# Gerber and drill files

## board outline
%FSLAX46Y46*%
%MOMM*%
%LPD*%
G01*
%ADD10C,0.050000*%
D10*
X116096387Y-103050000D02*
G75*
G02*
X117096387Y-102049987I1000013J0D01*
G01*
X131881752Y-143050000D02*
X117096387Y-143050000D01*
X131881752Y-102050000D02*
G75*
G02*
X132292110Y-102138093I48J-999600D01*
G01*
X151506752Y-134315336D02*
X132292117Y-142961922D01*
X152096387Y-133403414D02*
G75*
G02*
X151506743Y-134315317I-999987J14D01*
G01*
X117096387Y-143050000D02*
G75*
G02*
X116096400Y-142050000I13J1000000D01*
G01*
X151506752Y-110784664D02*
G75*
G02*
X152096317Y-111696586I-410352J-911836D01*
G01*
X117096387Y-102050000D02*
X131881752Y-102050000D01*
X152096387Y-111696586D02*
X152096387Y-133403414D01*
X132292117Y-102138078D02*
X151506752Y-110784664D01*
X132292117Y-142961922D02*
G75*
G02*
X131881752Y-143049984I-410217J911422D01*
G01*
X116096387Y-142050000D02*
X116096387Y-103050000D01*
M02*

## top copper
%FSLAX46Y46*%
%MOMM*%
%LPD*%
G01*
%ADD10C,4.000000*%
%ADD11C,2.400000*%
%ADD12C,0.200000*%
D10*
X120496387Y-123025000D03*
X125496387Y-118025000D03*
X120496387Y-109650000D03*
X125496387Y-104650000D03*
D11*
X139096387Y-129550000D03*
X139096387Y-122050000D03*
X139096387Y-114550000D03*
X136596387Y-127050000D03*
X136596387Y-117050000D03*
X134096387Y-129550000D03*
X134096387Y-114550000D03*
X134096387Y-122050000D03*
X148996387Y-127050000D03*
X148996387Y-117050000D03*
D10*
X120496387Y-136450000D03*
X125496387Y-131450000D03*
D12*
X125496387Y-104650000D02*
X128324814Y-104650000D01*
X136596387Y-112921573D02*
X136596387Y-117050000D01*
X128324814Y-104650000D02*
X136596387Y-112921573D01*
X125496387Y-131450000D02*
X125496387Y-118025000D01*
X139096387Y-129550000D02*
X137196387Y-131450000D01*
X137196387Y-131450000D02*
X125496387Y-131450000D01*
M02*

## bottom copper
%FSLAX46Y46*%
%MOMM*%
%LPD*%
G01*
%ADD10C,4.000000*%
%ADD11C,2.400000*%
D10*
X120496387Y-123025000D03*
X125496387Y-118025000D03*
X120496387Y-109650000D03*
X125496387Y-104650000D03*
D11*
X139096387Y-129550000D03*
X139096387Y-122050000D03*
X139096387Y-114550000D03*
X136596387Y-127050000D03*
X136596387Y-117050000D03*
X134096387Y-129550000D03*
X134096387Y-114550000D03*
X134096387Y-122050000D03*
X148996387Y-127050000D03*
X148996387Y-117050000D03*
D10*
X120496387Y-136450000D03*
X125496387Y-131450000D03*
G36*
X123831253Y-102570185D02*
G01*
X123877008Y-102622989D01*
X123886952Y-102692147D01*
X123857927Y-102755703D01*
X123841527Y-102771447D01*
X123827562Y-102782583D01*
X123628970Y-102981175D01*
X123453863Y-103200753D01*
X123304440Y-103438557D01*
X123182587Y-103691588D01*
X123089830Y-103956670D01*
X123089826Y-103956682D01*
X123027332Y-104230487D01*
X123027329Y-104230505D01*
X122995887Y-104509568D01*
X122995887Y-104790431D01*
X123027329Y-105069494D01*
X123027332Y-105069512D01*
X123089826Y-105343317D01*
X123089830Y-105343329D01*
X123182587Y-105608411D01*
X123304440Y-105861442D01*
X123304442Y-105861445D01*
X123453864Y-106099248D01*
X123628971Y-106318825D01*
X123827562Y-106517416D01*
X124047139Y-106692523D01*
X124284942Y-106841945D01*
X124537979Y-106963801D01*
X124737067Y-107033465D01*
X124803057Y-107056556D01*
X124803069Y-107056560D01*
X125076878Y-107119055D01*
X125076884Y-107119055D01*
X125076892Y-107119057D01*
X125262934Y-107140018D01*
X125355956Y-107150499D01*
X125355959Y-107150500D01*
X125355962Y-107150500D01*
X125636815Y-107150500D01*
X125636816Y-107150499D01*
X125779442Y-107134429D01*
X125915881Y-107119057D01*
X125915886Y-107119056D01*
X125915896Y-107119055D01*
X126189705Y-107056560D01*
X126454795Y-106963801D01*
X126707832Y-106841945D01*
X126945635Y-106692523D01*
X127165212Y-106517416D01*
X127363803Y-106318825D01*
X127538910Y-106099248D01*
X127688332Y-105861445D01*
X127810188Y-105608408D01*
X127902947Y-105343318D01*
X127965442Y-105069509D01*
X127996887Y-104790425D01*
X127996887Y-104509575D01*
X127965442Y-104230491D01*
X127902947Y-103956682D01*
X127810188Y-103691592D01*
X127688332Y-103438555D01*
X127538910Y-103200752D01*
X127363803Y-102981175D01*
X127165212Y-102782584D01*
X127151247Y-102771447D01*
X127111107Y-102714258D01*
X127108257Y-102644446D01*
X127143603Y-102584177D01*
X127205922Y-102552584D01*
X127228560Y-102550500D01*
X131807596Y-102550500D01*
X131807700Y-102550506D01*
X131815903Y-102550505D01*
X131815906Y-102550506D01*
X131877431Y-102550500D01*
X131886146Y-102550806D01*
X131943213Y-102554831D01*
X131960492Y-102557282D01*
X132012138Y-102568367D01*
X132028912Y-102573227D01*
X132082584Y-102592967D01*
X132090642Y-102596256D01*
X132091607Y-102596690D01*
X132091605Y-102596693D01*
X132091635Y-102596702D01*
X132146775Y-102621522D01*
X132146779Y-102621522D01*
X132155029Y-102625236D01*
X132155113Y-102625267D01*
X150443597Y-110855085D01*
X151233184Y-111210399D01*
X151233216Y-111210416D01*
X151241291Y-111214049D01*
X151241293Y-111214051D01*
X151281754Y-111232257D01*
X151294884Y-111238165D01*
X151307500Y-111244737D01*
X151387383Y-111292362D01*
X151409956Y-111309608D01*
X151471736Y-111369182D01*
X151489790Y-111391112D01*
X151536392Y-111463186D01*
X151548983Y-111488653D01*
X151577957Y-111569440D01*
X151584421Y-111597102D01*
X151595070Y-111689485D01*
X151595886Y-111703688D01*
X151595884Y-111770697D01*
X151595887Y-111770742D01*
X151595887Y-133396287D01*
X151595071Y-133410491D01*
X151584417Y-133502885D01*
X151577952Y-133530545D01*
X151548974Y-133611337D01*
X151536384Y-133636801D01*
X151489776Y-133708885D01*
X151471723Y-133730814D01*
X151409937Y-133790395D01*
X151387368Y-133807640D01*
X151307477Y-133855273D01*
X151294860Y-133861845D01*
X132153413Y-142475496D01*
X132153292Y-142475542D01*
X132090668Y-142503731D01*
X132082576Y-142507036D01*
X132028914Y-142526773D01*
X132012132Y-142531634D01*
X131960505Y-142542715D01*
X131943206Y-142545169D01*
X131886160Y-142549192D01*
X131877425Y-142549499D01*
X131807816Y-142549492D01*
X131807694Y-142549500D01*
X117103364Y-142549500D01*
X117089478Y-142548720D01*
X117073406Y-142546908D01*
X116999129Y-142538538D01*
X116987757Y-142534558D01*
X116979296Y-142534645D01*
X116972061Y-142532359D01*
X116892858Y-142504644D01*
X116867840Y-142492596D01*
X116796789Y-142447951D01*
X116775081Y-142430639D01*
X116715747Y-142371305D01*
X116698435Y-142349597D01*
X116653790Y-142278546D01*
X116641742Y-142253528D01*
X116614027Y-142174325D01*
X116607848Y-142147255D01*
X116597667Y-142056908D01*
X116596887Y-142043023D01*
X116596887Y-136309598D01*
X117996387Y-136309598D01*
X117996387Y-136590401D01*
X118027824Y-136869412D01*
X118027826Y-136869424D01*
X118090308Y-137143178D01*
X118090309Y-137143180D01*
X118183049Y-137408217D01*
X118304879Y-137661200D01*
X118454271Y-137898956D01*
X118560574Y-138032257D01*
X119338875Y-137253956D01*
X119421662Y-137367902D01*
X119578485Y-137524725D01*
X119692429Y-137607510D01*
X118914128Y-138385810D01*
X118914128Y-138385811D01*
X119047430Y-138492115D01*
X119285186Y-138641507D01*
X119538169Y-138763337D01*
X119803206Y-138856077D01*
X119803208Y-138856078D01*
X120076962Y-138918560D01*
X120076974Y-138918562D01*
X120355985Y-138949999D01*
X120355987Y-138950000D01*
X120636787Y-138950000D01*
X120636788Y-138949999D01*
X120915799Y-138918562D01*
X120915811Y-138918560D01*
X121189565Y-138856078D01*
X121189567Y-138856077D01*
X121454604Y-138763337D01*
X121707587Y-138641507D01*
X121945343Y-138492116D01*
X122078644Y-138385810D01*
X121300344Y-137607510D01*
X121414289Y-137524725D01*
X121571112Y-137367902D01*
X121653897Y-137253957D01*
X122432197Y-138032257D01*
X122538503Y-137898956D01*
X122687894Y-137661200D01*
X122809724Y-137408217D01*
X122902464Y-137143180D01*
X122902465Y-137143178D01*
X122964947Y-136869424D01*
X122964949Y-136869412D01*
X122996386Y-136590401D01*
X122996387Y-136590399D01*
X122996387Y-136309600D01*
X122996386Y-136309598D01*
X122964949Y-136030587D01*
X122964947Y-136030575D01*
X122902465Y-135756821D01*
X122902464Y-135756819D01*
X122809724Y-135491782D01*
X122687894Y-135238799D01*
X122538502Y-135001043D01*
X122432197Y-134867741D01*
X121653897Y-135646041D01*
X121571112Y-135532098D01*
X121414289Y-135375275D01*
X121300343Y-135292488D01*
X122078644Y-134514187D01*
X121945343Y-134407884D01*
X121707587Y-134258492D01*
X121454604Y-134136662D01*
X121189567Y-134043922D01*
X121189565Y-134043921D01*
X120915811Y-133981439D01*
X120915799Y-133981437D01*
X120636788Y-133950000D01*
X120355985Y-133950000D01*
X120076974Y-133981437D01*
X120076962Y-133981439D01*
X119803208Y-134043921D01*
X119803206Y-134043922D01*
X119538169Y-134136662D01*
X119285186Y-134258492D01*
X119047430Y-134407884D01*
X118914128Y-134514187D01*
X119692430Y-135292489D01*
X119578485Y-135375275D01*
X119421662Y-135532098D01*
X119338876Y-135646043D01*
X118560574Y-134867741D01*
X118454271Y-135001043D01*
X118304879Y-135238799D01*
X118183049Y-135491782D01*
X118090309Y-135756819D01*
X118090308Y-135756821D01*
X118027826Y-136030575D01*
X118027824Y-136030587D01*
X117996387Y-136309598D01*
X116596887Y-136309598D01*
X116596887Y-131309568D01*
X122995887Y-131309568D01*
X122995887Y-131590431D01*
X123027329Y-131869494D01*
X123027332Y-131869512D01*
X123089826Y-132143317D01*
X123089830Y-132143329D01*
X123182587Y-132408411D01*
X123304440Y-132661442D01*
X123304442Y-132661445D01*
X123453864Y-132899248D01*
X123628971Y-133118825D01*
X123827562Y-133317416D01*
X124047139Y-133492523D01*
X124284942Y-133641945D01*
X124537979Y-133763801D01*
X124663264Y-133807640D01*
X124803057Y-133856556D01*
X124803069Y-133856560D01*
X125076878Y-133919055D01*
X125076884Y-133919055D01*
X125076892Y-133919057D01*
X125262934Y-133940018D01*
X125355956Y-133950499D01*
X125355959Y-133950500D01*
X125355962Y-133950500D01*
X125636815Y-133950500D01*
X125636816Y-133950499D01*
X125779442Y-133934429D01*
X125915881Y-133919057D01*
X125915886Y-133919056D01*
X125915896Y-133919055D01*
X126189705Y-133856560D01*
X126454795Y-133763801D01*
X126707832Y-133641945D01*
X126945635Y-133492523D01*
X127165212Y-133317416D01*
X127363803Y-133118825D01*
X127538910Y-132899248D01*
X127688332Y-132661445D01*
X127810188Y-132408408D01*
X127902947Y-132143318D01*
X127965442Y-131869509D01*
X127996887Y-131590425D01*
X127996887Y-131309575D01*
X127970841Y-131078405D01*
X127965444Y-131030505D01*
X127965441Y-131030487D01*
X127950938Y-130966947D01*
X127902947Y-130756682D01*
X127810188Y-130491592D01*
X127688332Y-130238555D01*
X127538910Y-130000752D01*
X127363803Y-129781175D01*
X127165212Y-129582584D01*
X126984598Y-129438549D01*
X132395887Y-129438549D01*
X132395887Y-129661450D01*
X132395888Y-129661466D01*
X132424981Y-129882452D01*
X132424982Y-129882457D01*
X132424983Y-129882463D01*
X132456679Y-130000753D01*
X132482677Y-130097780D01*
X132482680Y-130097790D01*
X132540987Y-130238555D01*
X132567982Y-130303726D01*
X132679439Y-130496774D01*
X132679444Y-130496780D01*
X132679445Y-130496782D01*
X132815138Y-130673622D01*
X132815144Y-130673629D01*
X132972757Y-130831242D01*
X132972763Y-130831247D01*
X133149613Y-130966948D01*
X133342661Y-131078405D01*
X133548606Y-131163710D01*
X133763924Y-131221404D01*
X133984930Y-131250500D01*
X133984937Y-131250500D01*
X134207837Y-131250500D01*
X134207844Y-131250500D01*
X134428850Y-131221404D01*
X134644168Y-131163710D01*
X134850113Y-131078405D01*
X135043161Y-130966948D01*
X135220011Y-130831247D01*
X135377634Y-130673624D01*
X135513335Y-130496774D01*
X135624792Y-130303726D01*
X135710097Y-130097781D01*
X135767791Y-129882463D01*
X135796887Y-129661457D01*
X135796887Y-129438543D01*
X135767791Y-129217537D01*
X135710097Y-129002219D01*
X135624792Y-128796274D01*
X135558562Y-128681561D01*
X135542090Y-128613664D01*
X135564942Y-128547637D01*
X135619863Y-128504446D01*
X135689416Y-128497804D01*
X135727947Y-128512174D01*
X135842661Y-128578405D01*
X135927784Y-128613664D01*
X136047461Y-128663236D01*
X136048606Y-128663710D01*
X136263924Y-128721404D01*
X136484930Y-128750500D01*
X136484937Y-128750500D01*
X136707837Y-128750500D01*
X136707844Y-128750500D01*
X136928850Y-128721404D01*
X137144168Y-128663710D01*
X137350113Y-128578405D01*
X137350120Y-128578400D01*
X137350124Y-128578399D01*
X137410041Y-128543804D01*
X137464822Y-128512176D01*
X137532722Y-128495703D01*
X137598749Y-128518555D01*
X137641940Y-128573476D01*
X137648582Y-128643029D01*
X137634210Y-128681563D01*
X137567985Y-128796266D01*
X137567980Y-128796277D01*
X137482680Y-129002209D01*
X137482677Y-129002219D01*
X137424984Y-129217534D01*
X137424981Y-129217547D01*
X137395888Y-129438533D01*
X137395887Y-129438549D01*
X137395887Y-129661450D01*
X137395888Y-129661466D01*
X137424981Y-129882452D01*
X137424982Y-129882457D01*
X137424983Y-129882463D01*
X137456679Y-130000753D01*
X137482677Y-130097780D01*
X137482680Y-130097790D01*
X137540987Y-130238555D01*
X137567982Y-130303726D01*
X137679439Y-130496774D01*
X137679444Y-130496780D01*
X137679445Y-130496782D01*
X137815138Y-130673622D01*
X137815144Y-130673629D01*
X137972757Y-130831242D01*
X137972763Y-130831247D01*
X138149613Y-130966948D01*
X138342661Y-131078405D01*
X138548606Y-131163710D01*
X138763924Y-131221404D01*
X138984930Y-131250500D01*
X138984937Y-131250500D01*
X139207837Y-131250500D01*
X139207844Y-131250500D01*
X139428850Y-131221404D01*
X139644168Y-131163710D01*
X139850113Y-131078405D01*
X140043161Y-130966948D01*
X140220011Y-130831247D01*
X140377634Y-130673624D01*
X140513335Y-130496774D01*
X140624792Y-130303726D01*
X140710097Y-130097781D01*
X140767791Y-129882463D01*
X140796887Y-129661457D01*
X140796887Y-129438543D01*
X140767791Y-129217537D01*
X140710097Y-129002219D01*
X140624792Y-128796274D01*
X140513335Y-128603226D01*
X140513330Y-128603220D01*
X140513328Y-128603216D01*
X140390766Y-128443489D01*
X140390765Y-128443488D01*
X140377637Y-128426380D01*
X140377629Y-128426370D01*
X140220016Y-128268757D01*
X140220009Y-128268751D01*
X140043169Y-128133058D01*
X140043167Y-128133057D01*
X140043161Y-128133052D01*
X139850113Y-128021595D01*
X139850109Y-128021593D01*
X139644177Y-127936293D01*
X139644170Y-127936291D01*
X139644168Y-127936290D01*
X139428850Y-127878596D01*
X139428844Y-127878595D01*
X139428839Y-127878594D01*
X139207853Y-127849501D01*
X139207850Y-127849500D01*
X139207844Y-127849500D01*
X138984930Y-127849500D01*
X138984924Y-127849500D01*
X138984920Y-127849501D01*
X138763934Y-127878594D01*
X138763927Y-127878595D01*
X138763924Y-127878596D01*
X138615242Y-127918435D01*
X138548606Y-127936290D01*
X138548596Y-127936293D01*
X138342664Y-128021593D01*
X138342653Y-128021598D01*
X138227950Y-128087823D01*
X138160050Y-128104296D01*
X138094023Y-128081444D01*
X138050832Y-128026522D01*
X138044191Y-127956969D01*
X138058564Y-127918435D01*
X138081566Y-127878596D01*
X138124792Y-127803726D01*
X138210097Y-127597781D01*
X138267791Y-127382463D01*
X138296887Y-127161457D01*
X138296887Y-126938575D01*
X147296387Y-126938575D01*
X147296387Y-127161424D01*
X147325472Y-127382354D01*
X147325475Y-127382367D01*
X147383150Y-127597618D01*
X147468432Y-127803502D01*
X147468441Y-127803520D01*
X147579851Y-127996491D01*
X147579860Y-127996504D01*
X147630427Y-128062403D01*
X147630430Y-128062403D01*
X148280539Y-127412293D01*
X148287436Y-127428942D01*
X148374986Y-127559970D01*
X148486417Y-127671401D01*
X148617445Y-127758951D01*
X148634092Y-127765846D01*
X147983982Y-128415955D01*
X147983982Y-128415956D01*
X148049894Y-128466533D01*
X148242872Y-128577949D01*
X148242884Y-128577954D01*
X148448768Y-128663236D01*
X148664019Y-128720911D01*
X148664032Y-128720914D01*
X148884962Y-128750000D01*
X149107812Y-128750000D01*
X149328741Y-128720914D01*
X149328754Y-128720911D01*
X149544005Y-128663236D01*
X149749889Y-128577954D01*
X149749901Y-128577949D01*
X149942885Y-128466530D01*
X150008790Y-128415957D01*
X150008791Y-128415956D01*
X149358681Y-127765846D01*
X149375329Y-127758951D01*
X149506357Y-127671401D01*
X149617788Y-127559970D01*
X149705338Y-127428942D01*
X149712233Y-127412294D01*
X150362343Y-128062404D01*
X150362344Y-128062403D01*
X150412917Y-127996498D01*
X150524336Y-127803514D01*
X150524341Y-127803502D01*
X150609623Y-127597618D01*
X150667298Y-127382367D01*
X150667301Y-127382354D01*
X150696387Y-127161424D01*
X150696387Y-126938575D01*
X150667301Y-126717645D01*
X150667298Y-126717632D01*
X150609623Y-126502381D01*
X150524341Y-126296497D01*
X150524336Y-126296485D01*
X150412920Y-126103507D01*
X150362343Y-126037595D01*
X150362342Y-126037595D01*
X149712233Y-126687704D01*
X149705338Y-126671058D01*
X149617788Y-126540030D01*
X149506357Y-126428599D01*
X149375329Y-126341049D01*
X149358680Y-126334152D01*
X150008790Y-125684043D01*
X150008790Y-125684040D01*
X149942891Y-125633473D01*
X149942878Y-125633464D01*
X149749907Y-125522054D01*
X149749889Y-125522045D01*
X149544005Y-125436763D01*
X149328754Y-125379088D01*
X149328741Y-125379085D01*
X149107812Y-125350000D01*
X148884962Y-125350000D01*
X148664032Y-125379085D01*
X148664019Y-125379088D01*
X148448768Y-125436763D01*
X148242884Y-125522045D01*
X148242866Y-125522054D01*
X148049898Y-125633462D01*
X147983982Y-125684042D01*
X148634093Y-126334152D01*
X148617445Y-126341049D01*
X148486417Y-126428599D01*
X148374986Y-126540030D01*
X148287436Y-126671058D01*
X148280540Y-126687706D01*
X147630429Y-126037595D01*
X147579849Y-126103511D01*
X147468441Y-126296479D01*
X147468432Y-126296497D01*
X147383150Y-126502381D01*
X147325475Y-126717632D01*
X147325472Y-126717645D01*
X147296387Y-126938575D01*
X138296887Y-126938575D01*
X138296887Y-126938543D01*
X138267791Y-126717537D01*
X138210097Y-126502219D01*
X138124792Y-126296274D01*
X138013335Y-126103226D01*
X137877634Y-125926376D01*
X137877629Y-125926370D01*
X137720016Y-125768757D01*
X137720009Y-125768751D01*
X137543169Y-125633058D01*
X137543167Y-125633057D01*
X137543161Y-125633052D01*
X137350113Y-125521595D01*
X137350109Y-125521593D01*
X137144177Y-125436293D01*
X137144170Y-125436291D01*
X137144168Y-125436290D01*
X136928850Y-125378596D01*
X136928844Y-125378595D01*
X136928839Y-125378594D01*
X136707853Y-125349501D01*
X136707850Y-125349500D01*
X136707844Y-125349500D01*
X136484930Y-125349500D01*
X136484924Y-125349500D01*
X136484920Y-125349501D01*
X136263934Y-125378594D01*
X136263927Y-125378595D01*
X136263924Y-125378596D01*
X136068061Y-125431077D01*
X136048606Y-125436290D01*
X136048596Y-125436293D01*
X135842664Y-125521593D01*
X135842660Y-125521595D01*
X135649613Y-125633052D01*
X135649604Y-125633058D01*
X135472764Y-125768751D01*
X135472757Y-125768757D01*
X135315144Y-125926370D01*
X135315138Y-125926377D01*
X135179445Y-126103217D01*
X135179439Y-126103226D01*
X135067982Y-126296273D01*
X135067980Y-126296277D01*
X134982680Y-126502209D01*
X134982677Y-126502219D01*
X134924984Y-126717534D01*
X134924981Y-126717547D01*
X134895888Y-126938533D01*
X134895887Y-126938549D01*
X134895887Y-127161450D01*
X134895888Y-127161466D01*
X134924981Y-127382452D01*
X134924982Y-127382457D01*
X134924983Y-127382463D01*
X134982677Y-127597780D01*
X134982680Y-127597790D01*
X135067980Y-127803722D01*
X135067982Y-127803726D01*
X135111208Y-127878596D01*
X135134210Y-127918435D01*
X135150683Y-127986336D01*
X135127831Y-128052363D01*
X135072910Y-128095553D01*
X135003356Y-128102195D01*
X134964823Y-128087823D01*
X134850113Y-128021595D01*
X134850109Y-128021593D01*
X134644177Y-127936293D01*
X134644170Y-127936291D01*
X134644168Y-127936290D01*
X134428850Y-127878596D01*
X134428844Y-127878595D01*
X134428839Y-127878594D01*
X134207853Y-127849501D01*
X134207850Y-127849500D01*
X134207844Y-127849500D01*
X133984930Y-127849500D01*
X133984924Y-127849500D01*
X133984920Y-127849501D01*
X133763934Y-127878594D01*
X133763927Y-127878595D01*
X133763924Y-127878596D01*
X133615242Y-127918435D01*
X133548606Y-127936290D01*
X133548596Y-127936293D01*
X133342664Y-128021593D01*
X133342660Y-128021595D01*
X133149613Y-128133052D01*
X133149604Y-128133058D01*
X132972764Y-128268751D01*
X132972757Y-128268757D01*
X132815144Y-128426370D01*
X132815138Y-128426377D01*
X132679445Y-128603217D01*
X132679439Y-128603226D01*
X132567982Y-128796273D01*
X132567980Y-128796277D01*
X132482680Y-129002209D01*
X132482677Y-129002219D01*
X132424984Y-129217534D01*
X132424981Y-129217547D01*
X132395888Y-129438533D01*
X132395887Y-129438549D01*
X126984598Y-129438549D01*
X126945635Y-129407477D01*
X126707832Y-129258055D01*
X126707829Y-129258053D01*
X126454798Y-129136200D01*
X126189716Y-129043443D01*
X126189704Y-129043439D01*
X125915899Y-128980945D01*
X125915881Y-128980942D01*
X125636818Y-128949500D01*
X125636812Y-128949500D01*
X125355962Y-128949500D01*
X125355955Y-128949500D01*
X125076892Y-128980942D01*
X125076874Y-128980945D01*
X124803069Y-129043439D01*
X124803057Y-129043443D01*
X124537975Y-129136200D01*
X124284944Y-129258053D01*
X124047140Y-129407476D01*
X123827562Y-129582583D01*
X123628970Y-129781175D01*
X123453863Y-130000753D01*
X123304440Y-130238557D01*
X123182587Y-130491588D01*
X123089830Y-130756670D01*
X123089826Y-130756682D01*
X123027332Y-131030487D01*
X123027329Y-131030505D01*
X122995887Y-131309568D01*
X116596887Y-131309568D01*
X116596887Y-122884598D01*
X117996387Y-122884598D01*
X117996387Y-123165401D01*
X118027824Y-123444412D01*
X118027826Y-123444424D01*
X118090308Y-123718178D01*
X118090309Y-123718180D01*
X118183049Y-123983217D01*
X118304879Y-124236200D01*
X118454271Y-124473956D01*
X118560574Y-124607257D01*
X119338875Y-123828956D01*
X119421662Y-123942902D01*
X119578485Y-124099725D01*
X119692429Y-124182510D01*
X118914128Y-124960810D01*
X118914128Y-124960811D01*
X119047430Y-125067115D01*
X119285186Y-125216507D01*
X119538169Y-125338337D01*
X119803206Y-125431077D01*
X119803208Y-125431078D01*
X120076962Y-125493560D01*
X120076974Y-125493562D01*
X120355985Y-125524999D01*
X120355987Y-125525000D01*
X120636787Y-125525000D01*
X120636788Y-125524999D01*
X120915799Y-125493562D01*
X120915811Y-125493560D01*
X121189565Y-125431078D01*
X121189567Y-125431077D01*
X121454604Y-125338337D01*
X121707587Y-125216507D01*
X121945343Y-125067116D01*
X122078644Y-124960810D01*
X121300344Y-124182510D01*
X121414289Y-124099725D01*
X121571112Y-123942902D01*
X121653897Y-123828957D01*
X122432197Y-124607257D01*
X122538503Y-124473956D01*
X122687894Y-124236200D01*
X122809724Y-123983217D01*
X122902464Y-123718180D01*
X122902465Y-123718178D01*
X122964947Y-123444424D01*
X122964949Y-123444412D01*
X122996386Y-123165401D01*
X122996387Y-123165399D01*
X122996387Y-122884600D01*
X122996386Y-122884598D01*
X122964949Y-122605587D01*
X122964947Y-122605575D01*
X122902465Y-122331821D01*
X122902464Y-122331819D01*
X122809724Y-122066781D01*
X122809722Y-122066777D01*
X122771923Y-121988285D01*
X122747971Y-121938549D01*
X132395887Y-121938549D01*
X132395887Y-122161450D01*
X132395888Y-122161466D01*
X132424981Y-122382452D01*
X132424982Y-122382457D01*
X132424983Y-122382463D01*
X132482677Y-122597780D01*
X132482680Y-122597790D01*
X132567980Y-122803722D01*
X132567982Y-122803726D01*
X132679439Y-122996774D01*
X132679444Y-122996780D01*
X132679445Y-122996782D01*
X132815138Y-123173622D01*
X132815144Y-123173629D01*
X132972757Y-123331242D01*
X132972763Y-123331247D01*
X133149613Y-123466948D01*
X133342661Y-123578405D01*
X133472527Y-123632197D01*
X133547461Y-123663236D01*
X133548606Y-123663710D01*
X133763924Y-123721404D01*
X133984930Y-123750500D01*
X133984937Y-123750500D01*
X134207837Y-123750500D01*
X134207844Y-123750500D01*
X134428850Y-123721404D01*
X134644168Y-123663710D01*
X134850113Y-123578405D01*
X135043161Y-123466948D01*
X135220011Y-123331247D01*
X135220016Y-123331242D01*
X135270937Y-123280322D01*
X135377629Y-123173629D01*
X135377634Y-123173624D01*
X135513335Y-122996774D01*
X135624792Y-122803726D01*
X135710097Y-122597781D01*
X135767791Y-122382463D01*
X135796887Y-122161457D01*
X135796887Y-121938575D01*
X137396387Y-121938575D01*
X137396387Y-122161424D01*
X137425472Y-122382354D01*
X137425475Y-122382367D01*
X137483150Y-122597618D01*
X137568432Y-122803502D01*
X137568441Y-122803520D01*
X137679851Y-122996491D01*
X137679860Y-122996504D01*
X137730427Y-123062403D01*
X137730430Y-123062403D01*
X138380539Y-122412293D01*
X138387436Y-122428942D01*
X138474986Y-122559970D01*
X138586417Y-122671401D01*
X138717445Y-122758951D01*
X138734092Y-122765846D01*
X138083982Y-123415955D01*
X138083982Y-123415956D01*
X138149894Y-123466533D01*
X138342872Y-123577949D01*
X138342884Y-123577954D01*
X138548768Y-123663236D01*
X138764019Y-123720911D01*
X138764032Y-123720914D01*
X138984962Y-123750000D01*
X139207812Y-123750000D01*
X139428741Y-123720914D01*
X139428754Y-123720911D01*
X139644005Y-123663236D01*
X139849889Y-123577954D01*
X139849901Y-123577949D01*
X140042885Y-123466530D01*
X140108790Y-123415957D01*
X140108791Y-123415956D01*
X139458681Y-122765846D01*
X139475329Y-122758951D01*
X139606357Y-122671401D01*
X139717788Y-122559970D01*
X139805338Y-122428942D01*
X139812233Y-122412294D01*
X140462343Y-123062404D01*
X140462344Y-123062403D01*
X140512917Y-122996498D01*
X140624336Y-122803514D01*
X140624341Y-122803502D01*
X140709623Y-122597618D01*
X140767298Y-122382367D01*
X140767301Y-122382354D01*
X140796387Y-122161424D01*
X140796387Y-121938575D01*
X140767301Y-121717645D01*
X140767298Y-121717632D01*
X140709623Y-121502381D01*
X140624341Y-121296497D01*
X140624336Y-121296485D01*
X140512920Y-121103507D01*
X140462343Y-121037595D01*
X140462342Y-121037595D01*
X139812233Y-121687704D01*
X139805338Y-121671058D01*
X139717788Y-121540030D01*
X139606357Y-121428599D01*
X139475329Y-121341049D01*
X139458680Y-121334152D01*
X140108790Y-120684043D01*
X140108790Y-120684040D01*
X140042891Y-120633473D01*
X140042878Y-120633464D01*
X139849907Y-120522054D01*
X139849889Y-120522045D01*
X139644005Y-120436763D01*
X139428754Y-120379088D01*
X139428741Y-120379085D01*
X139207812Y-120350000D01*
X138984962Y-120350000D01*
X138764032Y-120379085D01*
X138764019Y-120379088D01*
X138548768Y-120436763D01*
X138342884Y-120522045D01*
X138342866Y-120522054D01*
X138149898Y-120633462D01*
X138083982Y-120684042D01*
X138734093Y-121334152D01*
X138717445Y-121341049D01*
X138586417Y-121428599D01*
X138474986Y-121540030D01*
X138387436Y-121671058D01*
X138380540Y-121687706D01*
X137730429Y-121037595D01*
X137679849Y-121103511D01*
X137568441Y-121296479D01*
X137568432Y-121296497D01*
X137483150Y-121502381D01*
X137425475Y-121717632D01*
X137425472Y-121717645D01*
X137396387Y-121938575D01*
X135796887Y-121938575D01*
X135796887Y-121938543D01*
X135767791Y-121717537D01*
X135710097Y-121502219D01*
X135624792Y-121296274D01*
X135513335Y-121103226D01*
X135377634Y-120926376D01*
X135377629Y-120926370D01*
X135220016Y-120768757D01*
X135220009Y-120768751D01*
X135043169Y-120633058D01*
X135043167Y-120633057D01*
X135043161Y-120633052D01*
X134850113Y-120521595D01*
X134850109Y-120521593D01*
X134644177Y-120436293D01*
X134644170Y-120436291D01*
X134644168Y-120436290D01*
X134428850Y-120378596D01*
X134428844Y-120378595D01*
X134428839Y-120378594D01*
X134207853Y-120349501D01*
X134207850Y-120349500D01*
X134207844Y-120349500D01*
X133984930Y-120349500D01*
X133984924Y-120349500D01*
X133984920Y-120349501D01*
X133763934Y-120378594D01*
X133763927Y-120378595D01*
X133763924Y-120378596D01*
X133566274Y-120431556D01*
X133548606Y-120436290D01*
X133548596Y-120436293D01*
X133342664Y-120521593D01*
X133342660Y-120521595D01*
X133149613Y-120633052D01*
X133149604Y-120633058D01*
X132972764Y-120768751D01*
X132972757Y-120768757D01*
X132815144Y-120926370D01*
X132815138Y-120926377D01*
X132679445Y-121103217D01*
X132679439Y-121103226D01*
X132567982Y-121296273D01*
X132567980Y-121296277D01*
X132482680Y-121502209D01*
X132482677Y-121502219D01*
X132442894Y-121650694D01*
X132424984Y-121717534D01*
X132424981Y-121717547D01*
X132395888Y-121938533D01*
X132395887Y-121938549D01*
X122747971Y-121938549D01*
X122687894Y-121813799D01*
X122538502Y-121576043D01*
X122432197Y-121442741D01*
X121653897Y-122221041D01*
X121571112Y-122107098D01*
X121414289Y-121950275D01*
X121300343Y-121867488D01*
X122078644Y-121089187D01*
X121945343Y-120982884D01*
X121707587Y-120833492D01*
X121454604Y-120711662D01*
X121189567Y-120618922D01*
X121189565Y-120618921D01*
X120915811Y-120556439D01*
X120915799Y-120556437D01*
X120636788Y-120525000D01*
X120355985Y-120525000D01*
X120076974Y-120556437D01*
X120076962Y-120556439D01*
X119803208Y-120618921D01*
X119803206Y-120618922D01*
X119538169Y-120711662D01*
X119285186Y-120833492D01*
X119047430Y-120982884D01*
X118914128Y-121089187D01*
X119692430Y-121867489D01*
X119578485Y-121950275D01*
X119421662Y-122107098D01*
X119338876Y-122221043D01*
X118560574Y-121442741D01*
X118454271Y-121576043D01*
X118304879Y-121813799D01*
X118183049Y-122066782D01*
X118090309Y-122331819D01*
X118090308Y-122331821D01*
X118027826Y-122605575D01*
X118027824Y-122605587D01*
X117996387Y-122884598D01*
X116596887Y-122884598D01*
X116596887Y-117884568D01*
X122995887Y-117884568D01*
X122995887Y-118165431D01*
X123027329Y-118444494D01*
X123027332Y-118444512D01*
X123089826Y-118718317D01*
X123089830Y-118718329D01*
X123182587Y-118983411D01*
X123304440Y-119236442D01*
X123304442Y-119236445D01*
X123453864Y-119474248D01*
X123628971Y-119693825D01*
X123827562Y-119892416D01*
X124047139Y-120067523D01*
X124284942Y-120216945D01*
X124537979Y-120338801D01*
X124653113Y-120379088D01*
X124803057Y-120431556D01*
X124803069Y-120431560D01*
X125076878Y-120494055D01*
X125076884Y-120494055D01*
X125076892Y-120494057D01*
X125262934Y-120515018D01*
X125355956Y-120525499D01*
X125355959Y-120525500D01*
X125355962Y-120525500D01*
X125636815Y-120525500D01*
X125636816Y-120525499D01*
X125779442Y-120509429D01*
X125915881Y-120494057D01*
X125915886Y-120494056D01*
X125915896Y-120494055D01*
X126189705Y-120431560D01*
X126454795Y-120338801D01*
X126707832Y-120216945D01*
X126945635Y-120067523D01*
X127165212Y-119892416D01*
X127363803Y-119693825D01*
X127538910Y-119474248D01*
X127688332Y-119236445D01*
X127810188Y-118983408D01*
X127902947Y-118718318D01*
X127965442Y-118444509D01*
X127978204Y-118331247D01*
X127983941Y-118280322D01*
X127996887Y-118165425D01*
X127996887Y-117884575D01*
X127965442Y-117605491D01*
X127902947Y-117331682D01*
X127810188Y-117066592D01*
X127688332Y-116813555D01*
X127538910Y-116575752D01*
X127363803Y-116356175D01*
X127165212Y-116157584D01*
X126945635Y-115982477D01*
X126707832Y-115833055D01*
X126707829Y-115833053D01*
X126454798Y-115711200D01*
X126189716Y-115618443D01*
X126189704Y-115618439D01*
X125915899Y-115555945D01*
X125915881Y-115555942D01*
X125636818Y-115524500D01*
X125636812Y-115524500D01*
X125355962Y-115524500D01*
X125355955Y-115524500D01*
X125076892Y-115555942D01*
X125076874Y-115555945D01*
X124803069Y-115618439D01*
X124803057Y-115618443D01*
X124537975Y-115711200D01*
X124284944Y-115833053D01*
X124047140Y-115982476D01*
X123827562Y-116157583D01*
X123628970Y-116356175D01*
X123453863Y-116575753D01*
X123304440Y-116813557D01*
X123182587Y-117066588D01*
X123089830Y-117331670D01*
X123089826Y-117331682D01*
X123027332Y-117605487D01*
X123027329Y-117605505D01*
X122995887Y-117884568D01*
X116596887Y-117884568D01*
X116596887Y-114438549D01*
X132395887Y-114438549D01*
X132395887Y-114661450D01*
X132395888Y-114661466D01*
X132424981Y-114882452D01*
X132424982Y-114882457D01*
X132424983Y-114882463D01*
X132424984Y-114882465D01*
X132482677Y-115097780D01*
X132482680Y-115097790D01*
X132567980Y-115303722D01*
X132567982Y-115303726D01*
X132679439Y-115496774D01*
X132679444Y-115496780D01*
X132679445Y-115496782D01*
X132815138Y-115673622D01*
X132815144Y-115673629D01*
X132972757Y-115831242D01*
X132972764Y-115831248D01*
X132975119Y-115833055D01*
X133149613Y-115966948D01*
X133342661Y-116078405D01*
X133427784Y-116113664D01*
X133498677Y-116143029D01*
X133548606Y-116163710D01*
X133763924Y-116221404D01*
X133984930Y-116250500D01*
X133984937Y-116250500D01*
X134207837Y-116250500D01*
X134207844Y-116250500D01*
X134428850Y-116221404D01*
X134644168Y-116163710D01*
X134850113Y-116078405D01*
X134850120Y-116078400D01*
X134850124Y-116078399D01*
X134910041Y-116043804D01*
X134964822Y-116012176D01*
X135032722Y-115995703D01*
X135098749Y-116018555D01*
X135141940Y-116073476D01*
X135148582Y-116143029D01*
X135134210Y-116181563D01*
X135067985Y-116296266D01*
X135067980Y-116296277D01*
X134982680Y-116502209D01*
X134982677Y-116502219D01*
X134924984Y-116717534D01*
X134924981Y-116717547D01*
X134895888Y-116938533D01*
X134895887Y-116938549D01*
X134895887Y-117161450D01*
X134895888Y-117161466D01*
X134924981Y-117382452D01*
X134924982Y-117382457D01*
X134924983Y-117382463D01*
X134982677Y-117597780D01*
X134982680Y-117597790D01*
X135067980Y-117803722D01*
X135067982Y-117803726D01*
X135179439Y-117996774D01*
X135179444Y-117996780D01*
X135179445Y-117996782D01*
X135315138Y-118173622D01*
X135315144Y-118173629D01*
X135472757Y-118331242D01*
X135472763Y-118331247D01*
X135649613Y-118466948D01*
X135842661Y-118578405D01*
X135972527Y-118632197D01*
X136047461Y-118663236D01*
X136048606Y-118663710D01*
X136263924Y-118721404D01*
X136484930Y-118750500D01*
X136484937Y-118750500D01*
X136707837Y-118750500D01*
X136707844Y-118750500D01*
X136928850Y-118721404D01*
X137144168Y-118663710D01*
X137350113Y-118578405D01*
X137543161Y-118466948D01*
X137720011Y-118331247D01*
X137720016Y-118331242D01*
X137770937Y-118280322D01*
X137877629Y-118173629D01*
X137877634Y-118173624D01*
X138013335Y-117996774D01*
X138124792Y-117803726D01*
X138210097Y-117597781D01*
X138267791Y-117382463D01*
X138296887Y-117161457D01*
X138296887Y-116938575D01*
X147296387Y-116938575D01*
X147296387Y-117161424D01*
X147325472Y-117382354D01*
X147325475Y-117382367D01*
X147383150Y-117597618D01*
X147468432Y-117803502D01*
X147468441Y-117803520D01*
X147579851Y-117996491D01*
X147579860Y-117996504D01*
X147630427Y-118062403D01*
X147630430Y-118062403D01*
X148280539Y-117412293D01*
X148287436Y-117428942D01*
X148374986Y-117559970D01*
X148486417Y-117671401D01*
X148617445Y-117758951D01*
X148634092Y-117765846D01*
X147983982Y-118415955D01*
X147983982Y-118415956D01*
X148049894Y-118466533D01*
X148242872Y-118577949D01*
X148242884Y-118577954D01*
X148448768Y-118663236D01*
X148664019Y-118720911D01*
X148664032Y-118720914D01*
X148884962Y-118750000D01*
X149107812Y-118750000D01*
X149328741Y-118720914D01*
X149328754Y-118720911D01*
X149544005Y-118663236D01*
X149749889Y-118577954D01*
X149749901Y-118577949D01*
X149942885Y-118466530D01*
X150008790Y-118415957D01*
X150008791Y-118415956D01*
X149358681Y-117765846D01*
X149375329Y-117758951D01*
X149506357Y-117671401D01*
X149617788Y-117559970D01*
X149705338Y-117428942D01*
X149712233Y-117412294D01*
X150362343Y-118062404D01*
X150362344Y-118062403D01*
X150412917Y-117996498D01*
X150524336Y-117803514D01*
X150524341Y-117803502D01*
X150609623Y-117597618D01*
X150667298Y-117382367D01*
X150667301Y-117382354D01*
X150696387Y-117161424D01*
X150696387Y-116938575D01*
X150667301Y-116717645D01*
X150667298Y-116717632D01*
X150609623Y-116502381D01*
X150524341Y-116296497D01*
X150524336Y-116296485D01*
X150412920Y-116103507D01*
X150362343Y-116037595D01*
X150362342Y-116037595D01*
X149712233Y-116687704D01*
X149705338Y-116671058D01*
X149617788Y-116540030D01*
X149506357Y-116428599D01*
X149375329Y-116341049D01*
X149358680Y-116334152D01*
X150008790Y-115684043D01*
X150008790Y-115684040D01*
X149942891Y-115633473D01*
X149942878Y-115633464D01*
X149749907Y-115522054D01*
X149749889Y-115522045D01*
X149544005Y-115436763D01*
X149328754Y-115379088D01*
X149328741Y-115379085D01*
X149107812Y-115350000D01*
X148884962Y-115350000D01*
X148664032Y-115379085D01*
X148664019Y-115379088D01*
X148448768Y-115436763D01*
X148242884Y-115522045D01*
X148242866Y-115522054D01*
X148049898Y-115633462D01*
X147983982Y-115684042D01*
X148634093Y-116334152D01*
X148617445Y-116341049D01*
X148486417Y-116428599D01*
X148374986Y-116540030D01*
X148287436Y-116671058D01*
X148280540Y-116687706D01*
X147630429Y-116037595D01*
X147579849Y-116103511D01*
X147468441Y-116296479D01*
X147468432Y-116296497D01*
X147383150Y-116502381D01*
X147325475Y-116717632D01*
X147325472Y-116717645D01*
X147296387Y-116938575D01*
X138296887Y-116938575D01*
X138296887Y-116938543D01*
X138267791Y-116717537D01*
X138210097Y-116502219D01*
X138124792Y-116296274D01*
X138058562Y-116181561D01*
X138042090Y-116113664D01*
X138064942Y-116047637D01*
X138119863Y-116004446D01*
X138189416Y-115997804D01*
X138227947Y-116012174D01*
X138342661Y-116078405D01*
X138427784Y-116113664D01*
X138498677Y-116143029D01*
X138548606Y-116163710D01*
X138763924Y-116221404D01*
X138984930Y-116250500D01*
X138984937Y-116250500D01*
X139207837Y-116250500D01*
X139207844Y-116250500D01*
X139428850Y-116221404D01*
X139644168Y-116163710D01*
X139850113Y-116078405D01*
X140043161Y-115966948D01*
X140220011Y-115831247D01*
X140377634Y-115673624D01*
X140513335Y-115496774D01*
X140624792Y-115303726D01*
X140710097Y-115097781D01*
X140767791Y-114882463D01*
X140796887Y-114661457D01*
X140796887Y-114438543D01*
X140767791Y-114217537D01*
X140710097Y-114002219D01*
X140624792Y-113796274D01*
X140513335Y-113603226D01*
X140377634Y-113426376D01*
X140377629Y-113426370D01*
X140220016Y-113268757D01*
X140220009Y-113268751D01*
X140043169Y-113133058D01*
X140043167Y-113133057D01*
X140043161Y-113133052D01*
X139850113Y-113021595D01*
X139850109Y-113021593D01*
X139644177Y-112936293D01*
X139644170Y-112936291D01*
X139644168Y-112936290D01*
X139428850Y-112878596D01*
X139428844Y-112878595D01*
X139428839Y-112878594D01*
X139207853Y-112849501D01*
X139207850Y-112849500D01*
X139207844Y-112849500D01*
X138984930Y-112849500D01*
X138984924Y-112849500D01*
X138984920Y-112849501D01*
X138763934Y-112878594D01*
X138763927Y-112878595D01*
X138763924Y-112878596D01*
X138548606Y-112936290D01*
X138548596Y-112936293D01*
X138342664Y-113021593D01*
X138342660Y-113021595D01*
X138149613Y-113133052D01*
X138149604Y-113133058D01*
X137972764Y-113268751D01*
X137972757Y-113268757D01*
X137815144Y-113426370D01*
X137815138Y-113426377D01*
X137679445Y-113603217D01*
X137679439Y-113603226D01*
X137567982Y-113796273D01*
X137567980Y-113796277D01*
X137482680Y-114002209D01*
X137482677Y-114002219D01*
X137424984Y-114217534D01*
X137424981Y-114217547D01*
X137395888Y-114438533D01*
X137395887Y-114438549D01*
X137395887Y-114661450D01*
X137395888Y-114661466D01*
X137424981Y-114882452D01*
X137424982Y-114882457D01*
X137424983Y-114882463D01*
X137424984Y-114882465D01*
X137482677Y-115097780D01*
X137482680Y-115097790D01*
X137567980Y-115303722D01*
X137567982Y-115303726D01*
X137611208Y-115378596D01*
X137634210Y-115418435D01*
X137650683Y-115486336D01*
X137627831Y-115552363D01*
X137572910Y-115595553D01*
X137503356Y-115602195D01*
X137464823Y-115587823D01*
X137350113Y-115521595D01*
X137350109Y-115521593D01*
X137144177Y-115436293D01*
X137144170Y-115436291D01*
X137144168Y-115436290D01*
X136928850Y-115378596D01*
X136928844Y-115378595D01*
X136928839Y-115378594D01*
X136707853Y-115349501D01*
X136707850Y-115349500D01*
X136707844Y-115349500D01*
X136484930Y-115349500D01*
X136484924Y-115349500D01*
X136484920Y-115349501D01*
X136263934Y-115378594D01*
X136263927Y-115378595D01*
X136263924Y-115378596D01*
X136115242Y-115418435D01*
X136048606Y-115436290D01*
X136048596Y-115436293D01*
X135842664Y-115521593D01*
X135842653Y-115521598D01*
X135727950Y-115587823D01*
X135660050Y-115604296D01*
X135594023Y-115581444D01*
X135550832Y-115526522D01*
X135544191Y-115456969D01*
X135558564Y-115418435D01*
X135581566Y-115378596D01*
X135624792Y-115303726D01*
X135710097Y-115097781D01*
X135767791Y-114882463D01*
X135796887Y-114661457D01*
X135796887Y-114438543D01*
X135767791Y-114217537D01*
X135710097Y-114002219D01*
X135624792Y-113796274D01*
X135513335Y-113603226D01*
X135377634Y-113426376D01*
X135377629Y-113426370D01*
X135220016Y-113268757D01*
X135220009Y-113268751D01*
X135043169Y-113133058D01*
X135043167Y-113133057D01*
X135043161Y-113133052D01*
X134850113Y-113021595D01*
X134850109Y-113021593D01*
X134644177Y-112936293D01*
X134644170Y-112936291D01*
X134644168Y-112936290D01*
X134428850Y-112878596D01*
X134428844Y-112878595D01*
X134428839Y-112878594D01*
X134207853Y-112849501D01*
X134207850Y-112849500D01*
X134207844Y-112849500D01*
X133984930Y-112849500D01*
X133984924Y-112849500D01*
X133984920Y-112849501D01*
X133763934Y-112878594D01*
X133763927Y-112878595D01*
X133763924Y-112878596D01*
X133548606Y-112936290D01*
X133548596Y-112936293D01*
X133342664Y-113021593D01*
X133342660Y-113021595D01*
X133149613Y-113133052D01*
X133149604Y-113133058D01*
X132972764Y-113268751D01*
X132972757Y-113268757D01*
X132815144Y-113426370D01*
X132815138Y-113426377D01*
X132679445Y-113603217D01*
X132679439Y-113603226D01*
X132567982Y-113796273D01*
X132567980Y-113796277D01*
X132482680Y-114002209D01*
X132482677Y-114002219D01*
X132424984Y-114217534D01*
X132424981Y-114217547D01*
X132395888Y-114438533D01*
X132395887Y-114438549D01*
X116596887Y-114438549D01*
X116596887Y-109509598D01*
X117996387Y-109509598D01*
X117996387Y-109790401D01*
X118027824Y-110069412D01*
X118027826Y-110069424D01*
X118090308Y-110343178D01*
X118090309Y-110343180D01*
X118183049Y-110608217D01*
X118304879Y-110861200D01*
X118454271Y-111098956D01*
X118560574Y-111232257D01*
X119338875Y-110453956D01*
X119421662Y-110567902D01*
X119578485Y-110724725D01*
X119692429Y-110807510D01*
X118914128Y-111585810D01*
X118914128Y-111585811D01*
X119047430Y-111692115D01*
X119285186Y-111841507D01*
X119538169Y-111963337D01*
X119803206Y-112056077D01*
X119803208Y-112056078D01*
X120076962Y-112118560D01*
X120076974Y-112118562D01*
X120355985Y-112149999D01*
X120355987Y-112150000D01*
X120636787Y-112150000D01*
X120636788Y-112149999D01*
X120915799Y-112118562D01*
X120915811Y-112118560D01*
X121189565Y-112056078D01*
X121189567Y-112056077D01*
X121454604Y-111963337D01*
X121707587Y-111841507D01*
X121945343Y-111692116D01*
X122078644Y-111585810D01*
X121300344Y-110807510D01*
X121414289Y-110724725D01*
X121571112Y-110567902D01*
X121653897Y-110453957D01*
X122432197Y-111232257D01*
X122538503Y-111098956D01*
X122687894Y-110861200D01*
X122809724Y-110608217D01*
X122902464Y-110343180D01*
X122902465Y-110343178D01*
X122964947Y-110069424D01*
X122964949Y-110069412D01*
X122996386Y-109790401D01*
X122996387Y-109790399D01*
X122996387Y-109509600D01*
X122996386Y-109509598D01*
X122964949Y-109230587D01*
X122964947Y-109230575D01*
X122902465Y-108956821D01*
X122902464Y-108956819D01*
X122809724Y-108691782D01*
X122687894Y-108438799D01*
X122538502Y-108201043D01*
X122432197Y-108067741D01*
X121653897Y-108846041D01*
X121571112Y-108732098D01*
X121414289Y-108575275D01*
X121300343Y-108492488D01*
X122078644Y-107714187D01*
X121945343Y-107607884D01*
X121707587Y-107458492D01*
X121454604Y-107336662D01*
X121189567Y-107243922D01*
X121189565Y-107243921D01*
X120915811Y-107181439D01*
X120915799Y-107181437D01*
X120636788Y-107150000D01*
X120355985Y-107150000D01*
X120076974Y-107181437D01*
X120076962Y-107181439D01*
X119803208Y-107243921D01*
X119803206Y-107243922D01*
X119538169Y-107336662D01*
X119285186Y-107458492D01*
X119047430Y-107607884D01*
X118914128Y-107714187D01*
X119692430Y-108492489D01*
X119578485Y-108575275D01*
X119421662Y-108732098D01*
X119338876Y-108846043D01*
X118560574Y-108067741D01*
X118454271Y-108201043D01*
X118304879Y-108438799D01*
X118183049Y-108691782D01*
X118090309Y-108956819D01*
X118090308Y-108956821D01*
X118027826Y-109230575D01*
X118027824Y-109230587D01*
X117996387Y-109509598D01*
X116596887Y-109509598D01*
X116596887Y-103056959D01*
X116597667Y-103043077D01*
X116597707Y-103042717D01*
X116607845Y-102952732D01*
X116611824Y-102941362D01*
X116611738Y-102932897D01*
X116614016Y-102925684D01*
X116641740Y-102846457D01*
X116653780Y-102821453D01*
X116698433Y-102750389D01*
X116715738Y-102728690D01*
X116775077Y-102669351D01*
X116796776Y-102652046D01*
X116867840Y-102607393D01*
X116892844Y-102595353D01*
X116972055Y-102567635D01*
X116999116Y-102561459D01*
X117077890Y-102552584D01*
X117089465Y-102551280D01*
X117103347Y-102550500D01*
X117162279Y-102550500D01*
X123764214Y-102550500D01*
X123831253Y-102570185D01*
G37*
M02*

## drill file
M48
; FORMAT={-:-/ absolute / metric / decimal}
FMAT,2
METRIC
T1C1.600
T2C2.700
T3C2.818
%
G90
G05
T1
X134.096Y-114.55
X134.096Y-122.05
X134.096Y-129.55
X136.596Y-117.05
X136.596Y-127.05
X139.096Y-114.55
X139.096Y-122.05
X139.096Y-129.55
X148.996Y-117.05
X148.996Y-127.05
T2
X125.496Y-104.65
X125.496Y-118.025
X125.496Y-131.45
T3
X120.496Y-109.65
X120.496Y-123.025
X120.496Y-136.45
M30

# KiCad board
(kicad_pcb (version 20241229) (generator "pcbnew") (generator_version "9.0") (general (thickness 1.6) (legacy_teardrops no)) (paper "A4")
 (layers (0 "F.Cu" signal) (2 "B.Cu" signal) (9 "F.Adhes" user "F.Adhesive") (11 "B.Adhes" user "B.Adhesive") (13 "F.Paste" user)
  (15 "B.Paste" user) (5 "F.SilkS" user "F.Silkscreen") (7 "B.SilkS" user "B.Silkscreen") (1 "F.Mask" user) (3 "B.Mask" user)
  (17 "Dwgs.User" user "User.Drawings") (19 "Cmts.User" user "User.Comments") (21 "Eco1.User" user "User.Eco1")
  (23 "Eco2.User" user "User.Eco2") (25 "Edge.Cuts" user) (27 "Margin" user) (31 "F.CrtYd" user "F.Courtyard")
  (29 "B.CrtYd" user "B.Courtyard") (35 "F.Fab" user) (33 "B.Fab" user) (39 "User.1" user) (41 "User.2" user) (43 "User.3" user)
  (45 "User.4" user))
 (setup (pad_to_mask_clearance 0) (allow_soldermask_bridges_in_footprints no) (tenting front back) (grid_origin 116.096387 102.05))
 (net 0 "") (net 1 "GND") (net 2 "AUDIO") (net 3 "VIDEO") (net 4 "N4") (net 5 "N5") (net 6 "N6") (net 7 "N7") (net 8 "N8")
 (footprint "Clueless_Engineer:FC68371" (layer "F.Cu") (at 120.496387 123.025)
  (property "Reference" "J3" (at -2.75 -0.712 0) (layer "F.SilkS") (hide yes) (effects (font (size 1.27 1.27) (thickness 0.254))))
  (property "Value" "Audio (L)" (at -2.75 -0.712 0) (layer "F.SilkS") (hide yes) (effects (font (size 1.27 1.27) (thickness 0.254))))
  (pad "1" thru_hole circle (at 0 0) (size 4 4) (drill 2.818) (layers "*.Cu" "*.Mask") (remove_unused_layers no) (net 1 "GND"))
  (pad "3" thru_hole circle (at 5 -5) (size 4 4) (drill 2.7) (layers "*.Cu" "*.Mask") (remove_unused_layers no) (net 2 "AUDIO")))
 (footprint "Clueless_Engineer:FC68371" (layer "F.Cu") (at 120.496387 109.65)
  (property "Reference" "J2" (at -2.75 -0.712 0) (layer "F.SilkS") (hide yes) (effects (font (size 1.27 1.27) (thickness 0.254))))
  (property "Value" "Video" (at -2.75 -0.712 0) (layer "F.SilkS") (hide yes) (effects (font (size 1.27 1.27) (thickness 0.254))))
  (pad "1" thru_hole circle (at 0 0) (size 4 4) (drill 2.818) (layers "*.Cu" "*.Mask") (remove_unused_layers no) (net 1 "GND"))
  (pad "3" thru_hole circle (at 5 -5) (size 4 4) (drill 2.7) (layers "*.Cu" "*.Mask") (remove_unused_layers no) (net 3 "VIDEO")))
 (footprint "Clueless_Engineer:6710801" (layer "F.Cu") (at 139.096387 129.55 -90)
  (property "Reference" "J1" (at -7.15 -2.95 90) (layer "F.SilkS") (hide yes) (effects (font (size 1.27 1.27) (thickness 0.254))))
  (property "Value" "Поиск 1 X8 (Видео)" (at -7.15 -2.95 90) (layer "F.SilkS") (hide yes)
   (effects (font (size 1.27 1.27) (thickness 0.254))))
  (pad "1" thru_hole circle (at 0 0 270) (size 2.4 2.4) (drill 1.6) (layers "*.Cu" "*.Mask") (remove_unused_layers no) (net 2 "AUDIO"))
  (pad "2" thru_hole circle (at -7.5 0 270) (size 2.4 2.4) (drill 1.6) (layers "*.Cu" "*.Mask") (remove_unused_layers no) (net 1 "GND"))
  (pad "3" thru_hole circle (at -15 0 270) (size 2.4 2.4) (drill 1.6) (layers "*.Cu" "*.Mask") (remove_unused_layers no) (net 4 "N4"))
  (pad "4" thru_hole circle (at -2.5 2.5 270) (size 2.4 2.4) (drill 1.6) (layers "*.Cu" "*.Mask") (remove_unused_layers no) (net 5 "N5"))
  (pad "5" thru_hole circle (at -12.5 2.5 270) (size 2.4 2.4) (drill 1.6) (layers "*.Cu" "*.Mask") (remove_unused_layers no) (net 3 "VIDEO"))
  (pad "6" thru_hole circle (at 0 5 270) (size 2.4 2.4) (drill 1.6) (layers "*.Cu" "*.Mask") (remove_unused_layers no) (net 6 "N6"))
  (pad "7" thru_hole circle (at -15 5 270) (size 2.4 2.4) (drill 1.6) (layers "*.Cu" "*.Mask") (remove_unused_layers no) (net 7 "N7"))
  (pad "8" thru_hole circle (at -7.5 5 270) (size 2.4 2.4) (drill 1.6) (layers "*.Cu" "*.Mask") (remove_unused_layers no) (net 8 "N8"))
  (pad "MH1" thru_hole circle (at -2.5 -9.9 270) (size 2.4 2.4) (drill 1.6) (layers "*.Cu" "*.Mask") (remove_unused_layers no) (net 1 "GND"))
  (pad "MH2" thru_hole circle (at -12.5 -9.9 270) (size 2.4 2.4) (drill 1.6) (layers "*.Cu" "*.Mask") (remove_unused_layers no)
   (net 1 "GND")))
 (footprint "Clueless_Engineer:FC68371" (layer "F.Cu") (at 120.496387 136.45)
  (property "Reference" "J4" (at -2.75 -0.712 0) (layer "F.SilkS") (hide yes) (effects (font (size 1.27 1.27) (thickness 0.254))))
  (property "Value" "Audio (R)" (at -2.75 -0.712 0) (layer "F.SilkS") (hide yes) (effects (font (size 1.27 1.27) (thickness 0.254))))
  (pad "1" thru_hole circle (at 0 0) (size 4 4) (drill 2.818) (layers "*.Cu" "*.Mask") (remove_unused_layers no) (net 1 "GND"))
  (pad "3" thru_hole circle (at 5 -5) (size 4 4) (drill 2.7) (layers "*.Cu" "*.Mask") (remove_unused_layers no) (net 2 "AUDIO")))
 (gr_arc (start 116.096387 103.05) (mid 116.38928 102.342893) (end 117.096387 102.05) (stroke (width 0.05) (type default))
  (layer "Edge.Cuts"))
 (gr_line (start 131.881752 143.05) (end 117.096387 143.05) (stroke (width 0.05) (type default)) (layer "Edge.Cuts"))
 (gr_arc (start 131.881752 102.05) (mid 132.09161 102.072258) (end 132.292117 102.138078) (stroke (width 0.05) (type default))
  (layer "Edge.Cuts"))
 (gr_line (start 151.506752 134.315336) (end 132.292117 142.961922) (stroke (width 0.05) (type default)) (layer "Edge.Cuts"))
 (gr_arc (start 152.096387 133.403414) (mid 151.936138 133.946385) (end 151.506752 134.315336) (stroke (width 0.05) (type default))
  (layer "Edge.Cuts"))
 (gr_arc (start 117.096387 143.05) (mid 116.389289 142.757102) (end 116.096387 142.05) (stroke (width 0.05) (type default))
  (layer "Edge.Cuts"))
 (gr_arc (start 151.506752 110.784664) (mid 151.93615 111.153611) (end 152.096387 111.696586) (stroke (width 0.05) (type default))
  (layer "Edge.Cuts"))
 (gr_line (start 117.096387 102.05) (end 131.881752 102.05) (stroke (width 0.05) (type default)) (layer "Edge.Cuts"))
 (gr_line (start 152.096387 111.696586) (end 152.096387 133.403414) (stroke (width 0.05) (type default)) (layer "Edge.Cuts"))
 (gr_line (start 132.292117 102.138078) (end 151.506752 110.784664) (stroke (width 0.05) (type default)) (layer "Edge.Cuts"))
 (gr_arc (start 132.292117 142.961922) (mid 132.091609 143.027743) (end 131.881752 143.05) (stroke (width 0.05) (type default))
  (layer "Edge.Cuts"))
 (gr_line (start 116.096387 142.05) (end 116.096387 103.05) (stroke (width 0.05) (type default)) (layer "Edge.Cuts"))
 (segment (start 125.496387 104.65) (end 128.324814 104.65) (width 0.2) (layer "F.Cu") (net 3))
 (segment (start 136.596387 112.921573) (end 136.596387 117.05) (width 0.2) (layer "F.Cu") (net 3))
 (segment (start 128.324814 104.65) (end 136.596387 112.921573) (width 0.2) (layer "F.Cu") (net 3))
 (segment (start 125.496387 131.45) (end 125.496387 118.025) (width 0.2) (layer "F.Cu") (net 2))
 (segment (start 139.096387 129.55) (end 137.196387 131.45) (width 0.2) (layer "F.Cu") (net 2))
 (segment (start 137.196387 131.45) (end 125.496387 131.45) (width 0.2) (layer "F.Cu") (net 2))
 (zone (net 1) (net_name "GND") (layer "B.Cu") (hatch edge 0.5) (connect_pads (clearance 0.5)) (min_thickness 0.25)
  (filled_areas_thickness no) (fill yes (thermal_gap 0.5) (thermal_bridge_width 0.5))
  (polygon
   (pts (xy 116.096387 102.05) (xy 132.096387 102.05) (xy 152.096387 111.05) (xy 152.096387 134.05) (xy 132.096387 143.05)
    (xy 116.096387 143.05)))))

